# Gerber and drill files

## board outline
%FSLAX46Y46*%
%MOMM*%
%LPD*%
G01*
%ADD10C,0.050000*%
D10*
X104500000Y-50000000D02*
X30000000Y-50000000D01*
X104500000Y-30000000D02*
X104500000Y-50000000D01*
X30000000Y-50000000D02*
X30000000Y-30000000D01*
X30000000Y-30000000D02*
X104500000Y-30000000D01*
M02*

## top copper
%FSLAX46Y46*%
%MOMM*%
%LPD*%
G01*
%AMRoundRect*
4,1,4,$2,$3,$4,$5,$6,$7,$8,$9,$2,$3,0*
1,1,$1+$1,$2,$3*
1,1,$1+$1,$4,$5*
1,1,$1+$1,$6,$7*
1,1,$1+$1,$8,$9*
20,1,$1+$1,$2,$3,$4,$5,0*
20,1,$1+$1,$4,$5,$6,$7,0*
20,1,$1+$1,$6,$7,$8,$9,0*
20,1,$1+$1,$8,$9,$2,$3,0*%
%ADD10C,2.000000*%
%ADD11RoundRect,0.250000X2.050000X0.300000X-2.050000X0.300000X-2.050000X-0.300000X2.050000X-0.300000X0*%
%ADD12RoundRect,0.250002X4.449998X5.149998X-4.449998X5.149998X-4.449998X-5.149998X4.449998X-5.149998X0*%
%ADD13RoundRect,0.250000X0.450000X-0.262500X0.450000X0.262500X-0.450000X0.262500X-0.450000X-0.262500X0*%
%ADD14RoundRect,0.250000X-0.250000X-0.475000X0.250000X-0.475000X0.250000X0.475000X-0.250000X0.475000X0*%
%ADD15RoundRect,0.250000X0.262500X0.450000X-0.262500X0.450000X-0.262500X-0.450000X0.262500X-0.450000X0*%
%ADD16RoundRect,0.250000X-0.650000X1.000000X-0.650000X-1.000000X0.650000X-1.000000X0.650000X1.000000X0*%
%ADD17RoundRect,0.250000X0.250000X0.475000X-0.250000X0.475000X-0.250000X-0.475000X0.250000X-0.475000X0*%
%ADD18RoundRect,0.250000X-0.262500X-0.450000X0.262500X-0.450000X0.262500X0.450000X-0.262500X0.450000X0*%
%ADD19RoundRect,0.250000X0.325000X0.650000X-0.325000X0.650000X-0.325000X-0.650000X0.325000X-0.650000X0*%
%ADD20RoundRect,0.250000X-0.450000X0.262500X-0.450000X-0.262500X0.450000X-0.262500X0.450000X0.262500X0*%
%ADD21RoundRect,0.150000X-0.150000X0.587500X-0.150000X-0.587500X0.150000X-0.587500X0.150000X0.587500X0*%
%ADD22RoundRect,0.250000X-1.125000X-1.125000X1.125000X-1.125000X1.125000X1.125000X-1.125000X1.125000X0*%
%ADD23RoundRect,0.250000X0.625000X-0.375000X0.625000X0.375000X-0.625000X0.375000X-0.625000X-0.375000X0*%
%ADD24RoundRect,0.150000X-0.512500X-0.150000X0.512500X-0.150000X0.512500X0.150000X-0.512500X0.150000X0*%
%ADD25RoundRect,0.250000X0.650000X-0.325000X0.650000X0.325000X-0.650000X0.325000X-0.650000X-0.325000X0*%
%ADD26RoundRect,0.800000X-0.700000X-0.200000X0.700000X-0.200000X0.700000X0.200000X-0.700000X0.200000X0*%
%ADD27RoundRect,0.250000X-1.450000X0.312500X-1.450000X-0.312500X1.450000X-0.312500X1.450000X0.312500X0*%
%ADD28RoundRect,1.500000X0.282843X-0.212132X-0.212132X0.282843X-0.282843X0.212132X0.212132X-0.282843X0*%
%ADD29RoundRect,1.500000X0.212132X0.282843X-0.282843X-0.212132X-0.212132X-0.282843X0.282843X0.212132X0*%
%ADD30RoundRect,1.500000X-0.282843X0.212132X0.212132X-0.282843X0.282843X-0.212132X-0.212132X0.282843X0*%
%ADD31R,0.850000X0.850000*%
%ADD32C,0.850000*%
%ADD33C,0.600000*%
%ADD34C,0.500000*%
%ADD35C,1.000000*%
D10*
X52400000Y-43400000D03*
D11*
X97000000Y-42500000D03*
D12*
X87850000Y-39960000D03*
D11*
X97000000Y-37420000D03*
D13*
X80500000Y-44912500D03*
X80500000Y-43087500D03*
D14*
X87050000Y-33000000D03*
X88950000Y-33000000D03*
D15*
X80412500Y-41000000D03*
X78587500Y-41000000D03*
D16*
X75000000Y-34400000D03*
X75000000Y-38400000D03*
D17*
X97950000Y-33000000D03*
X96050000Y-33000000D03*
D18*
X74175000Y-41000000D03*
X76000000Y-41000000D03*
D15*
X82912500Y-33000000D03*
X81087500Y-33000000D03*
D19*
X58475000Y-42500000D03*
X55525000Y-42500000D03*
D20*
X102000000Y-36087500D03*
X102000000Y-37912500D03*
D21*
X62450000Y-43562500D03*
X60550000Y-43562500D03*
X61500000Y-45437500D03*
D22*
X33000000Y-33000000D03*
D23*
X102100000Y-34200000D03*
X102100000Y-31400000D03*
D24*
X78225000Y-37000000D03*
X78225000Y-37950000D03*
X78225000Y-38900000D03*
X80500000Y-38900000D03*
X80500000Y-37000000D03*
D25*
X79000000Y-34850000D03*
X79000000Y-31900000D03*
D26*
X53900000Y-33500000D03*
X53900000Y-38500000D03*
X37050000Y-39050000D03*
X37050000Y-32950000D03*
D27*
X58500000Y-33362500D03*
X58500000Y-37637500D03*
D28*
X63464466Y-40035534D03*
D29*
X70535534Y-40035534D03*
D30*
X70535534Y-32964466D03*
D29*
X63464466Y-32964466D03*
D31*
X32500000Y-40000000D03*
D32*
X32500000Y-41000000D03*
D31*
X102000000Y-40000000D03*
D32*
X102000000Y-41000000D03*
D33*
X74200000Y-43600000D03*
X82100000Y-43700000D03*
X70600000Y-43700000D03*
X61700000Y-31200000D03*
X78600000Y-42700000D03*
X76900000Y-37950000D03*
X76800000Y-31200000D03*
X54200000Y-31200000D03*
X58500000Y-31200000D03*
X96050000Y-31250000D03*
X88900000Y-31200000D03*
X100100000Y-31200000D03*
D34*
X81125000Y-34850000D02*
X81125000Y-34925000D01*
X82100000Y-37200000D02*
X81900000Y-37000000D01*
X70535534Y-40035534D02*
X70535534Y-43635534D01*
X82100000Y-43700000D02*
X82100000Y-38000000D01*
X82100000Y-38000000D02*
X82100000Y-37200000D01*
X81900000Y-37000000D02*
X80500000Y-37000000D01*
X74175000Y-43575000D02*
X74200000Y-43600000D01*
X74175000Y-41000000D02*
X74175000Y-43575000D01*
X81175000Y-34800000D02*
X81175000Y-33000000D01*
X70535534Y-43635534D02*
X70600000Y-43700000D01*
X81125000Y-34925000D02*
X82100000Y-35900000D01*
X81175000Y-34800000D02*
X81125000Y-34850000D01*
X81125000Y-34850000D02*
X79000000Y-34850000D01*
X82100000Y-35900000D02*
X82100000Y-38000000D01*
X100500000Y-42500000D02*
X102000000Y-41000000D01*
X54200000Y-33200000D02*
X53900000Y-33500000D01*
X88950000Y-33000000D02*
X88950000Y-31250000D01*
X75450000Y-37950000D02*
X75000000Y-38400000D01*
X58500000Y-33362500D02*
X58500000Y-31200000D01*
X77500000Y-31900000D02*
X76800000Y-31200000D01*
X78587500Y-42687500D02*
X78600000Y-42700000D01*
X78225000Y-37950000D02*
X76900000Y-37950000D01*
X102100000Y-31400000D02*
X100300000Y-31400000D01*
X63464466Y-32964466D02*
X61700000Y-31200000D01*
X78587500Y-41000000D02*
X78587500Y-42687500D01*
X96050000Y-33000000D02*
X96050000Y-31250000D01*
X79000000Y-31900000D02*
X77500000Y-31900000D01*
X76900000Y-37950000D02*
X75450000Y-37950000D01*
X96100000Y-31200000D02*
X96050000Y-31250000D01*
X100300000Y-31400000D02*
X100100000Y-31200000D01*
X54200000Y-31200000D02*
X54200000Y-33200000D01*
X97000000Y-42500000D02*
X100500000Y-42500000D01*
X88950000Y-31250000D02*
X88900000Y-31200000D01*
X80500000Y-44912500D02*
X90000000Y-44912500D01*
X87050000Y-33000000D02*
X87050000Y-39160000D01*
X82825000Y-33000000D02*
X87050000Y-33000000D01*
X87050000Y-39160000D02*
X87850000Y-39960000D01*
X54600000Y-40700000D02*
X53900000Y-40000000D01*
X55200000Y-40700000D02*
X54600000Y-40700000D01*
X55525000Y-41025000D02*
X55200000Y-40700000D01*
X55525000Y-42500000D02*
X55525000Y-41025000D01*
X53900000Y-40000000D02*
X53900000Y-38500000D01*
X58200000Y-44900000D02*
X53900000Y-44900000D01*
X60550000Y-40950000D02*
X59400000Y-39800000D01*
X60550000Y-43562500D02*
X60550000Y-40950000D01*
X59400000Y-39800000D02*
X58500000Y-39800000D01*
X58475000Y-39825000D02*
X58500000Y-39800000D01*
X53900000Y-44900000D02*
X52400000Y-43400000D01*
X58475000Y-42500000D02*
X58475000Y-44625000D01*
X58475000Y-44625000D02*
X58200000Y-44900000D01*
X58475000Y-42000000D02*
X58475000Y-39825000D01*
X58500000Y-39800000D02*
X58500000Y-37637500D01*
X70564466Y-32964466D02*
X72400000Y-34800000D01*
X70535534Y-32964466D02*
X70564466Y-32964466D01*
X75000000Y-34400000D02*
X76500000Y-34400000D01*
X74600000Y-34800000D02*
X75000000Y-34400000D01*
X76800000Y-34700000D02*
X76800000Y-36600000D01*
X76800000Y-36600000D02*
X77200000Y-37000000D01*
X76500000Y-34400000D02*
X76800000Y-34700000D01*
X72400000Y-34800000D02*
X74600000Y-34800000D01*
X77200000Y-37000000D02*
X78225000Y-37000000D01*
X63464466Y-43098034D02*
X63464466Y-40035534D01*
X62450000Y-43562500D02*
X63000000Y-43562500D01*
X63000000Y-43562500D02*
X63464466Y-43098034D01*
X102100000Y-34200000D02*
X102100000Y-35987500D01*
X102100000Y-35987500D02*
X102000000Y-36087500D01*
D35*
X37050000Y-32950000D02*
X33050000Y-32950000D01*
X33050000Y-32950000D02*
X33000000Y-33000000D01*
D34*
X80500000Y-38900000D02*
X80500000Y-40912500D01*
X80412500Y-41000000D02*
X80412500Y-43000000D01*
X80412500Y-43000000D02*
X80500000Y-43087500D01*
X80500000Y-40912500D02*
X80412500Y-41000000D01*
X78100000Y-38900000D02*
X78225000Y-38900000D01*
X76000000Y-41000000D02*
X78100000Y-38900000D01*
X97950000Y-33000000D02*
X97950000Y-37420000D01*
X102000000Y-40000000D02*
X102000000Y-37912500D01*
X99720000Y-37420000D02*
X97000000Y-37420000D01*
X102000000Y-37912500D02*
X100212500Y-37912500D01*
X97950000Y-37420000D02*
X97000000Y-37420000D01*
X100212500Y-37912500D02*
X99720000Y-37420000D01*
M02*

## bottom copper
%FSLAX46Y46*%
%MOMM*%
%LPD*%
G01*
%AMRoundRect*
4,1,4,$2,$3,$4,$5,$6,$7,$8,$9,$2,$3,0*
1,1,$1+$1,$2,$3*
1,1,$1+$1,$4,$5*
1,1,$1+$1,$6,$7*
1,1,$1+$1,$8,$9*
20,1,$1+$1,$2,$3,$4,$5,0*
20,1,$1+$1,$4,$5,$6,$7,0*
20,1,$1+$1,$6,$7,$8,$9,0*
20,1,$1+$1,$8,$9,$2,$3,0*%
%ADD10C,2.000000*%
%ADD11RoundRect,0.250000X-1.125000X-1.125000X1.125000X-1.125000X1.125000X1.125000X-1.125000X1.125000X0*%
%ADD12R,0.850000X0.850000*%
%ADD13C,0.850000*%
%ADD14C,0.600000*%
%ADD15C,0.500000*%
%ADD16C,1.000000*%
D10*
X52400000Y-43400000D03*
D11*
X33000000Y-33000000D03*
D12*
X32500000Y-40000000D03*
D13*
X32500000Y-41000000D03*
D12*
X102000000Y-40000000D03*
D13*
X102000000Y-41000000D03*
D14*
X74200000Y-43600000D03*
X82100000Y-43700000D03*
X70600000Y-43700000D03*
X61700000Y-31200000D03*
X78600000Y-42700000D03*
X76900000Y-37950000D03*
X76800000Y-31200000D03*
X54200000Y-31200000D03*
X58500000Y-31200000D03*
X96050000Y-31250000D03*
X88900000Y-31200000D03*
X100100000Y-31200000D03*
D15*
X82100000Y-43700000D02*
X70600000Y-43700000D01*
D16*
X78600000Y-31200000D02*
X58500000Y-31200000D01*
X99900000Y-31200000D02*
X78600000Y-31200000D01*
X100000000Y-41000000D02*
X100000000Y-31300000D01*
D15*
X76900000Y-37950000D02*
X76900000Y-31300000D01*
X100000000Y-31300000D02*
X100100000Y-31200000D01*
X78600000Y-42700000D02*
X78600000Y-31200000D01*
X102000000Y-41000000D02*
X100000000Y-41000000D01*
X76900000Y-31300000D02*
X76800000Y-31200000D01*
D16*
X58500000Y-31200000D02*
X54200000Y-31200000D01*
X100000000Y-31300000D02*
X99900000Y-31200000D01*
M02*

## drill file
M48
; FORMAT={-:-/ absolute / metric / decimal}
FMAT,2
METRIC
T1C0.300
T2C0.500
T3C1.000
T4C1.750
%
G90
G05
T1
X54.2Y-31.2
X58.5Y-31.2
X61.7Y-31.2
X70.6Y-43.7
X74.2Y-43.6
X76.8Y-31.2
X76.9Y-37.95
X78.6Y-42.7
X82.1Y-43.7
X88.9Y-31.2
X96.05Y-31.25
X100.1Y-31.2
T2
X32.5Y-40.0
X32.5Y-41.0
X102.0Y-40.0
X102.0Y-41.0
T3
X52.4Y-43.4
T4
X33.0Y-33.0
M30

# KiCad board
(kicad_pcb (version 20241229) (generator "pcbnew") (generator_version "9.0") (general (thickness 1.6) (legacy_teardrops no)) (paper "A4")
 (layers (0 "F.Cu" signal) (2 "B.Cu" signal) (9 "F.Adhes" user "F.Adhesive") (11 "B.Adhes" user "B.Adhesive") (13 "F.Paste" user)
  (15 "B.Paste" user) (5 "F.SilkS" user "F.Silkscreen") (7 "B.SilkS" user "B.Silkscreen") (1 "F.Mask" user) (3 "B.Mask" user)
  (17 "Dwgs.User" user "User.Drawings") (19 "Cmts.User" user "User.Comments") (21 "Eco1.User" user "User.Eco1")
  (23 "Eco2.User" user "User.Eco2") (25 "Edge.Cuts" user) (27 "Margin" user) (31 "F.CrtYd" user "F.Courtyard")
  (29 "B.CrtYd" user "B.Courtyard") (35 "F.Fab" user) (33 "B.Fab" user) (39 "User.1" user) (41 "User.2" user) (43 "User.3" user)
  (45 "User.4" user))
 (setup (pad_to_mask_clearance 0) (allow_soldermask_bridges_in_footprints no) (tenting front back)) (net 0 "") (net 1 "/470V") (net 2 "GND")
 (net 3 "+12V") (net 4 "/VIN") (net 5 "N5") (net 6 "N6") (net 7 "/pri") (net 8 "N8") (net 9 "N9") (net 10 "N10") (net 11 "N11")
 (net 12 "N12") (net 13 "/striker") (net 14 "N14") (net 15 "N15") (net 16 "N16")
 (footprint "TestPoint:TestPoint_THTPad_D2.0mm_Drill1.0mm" (layer "F.Cu") (at 52.4 43.4)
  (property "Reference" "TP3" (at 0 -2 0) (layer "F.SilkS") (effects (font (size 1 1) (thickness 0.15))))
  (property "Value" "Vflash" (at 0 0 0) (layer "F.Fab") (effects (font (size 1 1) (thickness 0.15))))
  (pad "1" thru_hole circle (at 0 0) (size 2 2) (drill 1) (layers "*.Cu" "*.Mask") (remove_unused_layers no) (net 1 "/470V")))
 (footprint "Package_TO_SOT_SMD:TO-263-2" (layer "F.Cu") (at 89.35 39.96 180)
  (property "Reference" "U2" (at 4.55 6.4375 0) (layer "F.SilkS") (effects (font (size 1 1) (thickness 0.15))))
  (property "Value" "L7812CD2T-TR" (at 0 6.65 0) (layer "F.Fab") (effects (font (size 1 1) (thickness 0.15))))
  (pad "" smd roundrect (at -0.925 -2.775 180) (size 4.55 5.25) (layers "F.Paste") (roundrect_rratio 0.054945))
  (pad "" smd roundrect (at -0.925 2.775 180) (size 4.55 5.25) (layers "F.Paste") (roundrect_rratio 0.054945))
  (pad "" smd roundrect (at 3.925 -2.775 180) (size 4.55 5.25) (layers "F.Paste") (roundrect_rratio 0.054945))
  (pad "" smd roundrect (at 3.925 2.775 180) (size 4.55 5.25) (layers "F.Paste") (roundrect_rratio 0.054945))
  (pad "1" smd roundrect (at -7.65 -2.54 180) (size 4.6 1.1) (layers "F.Cu" "F.Mask" "F.Paste") (roundrect_rratio 0.227273) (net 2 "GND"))
  (pad "2" smd roundrect (at 1.5 0 180) (size 9.4 10.8) (layers "F.Cu" "F.Mask") (roundrect_rratio 0.026596) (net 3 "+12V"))
  (pad "3" smd roundrect (at -7.65 2.54 180) (size 4.6 1.1) (layers "F.Cu" "F.Mask" "F.Paste") (roundrect_rratio 0.227273) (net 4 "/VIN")))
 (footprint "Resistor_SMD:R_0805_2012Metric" (layer "F.Cu") (at 80.5 44 90)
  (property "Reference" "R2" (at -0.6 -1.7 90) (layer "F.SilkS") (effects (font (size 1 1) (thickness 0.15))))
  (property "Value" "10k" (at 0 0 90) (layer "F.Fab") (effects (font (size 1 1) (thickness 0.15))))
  (pad "1" smd roundrect (at -0.9125 0 90) (size 1.025 1.4) (layers "F.Cu" "F.Mask" "F.Paste") (roundrect_rratio 0.243902) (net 3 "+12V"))
  (pad "2" smd roundrect (at 0.9125 0 90) (size 1.025 1.4) (layers "F.Cu" "F.Mask" "F.Paste") (roundrect_rratio 0.243902) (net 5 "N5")))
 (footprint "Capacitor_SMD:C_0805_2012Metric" (layer "F.Cu") (at 88 33)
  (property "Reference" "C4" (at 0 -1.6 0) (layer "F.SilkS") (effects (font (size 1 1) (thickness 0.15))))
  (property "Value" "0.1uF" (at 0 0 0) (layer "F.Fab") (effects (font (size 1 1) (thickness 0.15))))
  (pad "1" smd roundrect (at -0.95 0) (size 1 1.45) (layers "F.Cu" "F.Mask" "F.Paste") (roundrect_rratio 0.25) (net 3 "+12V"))
  (pad "2" smd roundrect (at 0.95 0) (size 1 1.45) (layers "F.Cu" "F.Mask" "F.Paste") (roundrect_rratio 0.25) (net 2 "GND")))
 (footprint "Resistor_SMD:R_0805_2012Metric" (layer "F.Cu") (at 79.5 41 180)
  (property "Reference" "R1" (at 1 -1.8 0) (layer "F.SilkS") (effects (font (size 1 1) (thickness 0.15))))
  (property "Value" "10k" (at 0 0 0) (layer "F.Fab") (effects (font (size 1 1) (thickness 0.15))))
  (pad "1" smd roundrect (at -0.9125 0 180) (size 1.025 1.4) (layers "F.Cu" "F.Mask" "F.Paste") (roundrect_rratio 0.243902) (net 5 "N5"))
  (pad "2" smd roundrect (at 0.9125 0 180) (size 1.025 1.4) (layers "F.Cu" "F.Mask" "F.Paste") (roundrect_rratio 0.243902) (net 2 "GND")))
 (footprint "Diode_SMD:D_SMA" (layer "F.Cu") (at 75 36.4 -90)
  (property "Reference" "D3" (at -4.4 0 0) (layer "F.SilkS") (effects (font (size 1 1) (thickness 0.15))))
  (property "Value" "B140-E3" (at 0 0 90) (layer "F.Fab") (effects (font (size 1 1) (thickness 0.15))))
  (pad "1" smd roundrect (at -2 0 270) (size 2.5 1.8) (layers "F.Cu" "F.Mask" "F.Paste") (roundrect_rratio 0.1388888889) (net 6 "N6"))
  (pad "2" smd roundrect (at 2 0 270) (size 2.5 1.8) (layers "F.Cu" "F.Mask" "F.Paste") (roundrect_rratio 0.1388888889) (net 2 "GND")))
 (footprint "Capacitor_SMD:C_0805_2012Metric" (layer "F.Cu") (at 97 33 180)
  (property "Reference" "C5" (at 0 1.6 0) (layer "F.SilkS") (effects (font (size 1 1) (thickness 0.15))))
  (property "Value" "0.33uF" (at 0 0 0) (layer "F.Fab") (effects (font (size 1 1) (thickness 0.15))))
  (pad "1" smd roundrect (at -0.95 0 180) (size 1 1.45) (layers "F.Cu" "F.Mask" "F.Paste") (roundrect_rratio 0.25) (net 4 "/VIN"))
  (pad "2" smd roundrect (at 0.95 0 180) (size 1 1.45) (layers "F.Cu" "F.Mask" "F.Paste") (roundrect_rratio 0.25) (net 2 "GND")))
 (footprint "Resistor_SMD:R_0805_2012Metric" (layer "F.Cu") (at 75.0875 41)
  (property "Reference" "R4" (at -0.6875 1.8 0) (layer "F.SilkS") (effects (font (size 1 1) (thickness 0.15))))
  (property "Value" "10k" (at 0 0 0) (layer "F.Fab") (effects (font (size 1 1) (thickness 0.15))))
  (pad "1" smd roundrect (at -0.9125 0) (size 1.025 1.4) (layers "F.Cu" "F.Mask" "F.Paste") (roundrect_rratio 0.243902) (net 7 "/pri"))
  (pad "2" smd roundrect (at 0.9125 0) (size 1.025 1.4) (layers "F.Cu" "F.Mask" "F.Paste") (roundrect_rratio 0.243902) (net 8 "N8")))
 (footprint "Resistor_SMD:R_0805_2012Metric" (layer "F.Cu") (at 82 33 180)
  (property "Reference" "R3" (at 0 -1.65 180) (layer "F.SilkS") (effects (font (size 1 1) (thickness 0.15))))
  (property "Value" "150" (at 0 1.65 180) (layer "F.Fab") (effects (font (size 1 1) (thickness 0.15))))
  (pad "1" smd roundrect (at -0.9125 0 180) (size 1.025 1.4) (layers "F.Cu" "F.Mask" "F.Paste") (roundrect_rratio 0.243902) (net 3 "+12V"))
  (pad "2" smd roundrect (at 0.9125 0 180) (size 1.025 1.4) (layers "F.Cu" "F.Mask" "F.Paste") (roundrect_rratio 0.243902) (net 7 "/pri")))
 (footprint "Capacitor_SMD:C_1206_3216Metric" (layer "F.Cu") (at 57 42.5 180)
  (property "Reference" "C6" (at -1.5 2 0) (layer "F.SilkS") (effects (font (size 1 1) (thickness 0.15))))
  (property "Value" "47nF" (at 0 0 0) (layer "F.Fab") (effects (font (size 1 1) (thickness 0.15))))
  (pad "1" smd roundrect (at -1.475 0 180) (size 1.15 1.8) (layers "F.Cu" "F.Mask" "F.Paste") (roundrect_rratio 0.217391) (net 1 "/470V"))
  (pad "2" smd roundrect (at 1.475 0 180) (size 1.15 1.8) (layers "F.Cu" "F.Mask" "F.Paste") (roundrect_rratio 0.217391) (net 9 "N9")))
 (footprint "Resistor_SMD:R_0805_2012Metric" (layer "F.Cu") (at 102 37 -90)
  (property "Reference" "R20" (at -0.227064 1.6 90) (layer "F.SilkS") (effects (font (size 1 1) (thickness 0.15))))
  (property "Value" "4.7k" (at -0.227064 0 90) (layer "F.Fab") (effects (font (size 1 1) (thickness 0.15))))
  (pad "1" smd roundrect (at -0.9125 0 270) (size 1.025 1.4) (layers "F.Cu" "F.Mask" "F.Paste") (roundrect_rratio 0.243902) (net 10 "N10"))
  (pad "2" smd roundrect (at 0.9125 0 270) (size 1.025 1.4) (layers "F.Cu" "F.Mask" "F.Paste") (roundrect_rratio 0.243902) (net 4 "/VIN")))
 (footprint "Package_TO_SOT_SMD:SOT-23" (layer "F.Cu") (at 61.5 44.5 -90)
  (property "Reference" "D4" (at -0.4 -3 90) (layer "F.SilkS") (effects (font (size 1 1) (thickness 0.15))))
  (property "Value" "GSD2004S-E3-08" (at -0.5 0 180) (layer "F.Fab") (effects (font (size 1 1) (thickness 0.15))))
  (pad "1" smd roundrect (at -0.9375 -0.95 270) (size 1.475 0.6) (layers "F.Cu" "F.Mask" "F.Paste") (roundrect_rratio 0.25) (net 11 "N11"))
  (pad "2" smd roundrect (at -0.9375 0.95 270) (size 1.475 0.6) (layers "F.Cu" "F.Mask" "F.Paste") (roundrect_rratio 0.25) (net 1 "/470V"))
  (pad "3" smd roundrect (at 0.9375 0 270) (size 1.475 0.6) (layers "F.Cu" "F.Mask" "F.Paste") (roundrect_rratio 0.25) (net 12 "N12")))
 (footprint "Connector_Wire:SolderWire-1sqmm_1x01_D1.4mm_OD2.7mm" (layer "F.Cu") (at 33 33)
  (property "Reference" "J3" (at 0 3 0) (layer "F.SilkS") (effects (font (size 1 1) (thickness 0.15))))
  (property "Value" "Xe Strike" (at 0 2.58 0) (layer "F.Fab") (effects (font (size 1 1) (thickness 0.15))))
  (pad "1" thru_hole roundrect (at 0 0) (size 2.75 2.75) (drill 1.75) (layers "*.Cu" "*.Mask") (remove_unused_layers no)
   (roundrect_rratio 0.090909) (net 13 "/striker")))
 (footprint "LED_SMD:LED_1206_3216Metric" (layer "F.Cu") (at 102.1 32.8 90)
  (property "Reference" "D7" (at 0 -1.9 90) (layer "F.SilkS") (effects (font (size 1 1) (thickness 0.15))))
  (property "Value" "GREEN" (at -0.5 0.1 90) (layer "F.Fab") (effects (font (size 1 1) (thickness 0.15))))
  (pad "1" smd roundrect (at -1.4 0 90) (size 1.25 1.75) (layers "F.Cu" "F.Mask" "F.Paste") (roundrect_rratio 0.2) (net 10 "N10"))
  (pad "2" smd roundrect (at 1.4 0 90) (size 1.25 1.75) (layers "F.Cu" "F.Mask" "F.Paste") (roundrect_rratio 0.2) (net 2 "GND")))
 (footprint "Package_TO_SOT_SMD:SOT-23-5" (layer "F.Cu") (at 79.3625 37.95)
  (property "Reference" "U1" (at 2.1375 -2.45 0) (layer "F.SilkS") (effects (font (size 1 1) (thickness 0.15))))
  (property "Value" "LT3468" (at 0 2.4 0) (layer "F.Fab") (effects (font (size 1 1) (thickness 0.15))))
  (pad "1" smd roundrect (at -1.1375 -0.95) (size 1.325 0.6) (layers "F.Cu" "F.Mask" "F.Paste") (roundrect_rratio 0.25) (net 6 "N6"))
  (pad "2" smd roundrect (at -1.1375 0) (size 1.325 0.6) (layers "F.Cu" "F.Mask" "F.Paste") (roundrect_rratio 0.25) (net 2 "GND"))
  (pad "3" smd roundrect (at -1.1375 0.95) (size 1.325 0.6) (layers "F.Cu" "F.Mask" "F.Paste") (roundrect_rratio 0.25) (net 8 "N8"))
  (pad "4" smd roundrect (at 1.1375 0.95) (size 1.325 0.6) (layers "F.Cu" "F.Mask" "F.Paste") (roundrect_rratio 0.25) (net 5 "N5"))
  (pad "5" smd roundrect (at 1.1375 -0.95) (size 1.325 0.6) (layers "F.Cu" "F.Mask" "F.Paste") (roundrect_rratio 0.25) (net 7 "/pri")))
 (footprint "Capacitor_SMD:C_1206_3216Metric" (layer "F.Cu") (at 79 33.375 90)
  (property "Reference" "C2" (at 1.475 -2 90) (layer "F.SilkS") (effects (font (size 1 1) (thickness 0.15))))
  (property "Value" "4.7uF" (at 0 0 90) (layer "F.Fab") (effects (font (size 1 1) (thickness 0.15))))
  (pad "1" smd roundrect (at -1.475 0 90) (size 1.15 1.8) (layers "F.Cu" "F.Mask" "F.Paste") (roundrect_rratio 0.217391) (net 7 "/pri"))
  (pad "2" smd roundrect (at 1.475 0 90) (size 1.15 1.8) (layers "F.Cu" "F.Mask" "F.Paste") (roundrect_rratio 0.217391) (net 2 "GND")))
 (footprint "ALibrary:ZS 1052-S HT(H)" (layer "F.Cu") (at 45.5 36 180)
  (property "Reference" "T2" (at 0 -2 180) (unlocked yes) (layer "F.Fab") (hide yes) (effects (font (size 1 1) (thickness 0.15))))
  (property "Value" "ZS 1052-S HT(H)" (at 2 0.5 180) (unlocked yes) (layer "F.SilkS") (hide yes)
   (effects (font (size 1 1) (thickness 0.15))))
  (pad "1" smd roundrect (at -8.4 2.5) (size 3 2) (layers "F.Cu" "F.Mask" "F.Paste") (roundrect_rratio 0.4) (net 2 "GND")
   (thermal_bridge_angle 45))
  (pad "2" smd roundrect (at -8.4 -2.5) (size 3 2) (layers "F.Cu" "F.Mask" "F.Paste") (roundrect_rratio 0.4) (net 9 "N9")
   (thermal_bridge_angle 45))
  (pad "3" smd roundrect (at 8.45 -3.05) (size 3 2) (layers "F.Cu" "F.Mask" "F.Paste") (roundrect_rratio 0.4) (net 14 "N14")
   (thermal_bridge_angle 45))
  (pad "4" smd roundrect (at 8.45 3.05) (size 3 2) (layers "F.Cu" "F.Mask" "F.Paste") (roundrect_rratio 0.4) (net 13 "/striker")
   (thermal_bridge_angle 45)))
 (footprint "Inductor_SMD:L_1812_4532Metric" (layer "F.Cu") (at 58.5 35.5 -90)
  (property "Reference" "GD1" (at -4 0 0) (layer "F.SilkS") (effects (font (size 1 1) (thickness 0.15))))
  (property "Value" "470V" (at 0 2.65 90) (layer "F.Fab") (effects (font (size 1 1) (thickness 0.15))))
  (pad "1" smd roundrect (at -2.1375 0 270) (size 1.125 3.4) (layers "F.Cu" "F.Mask" "F.Paste") (roundrect_rratio 0.222222) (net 2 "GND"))
  (pad "2" smd roundrect (at 2.1375 0 270) (size 1.125 3.4) (layers "F.Cu" "F.Mask" "F.Paste") (roundrect_rratio 0.222222) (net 1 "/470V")))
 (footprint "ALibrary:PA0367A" (layer "F.Cu") (at 67 36.5 135)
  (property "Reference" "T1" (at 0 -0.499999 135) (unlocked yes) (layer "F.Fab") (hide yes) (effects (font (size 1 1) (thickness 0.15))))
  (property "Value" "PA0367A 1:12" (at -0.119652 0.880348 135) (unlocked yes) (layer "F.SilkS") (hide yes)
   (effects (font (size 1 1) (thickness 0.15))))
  (pad "1" smd roundrect (at 0 -5 135) (size 3.7 3.1) (layers "F.Cu" "F.Mask" "F.Paste") (roundrect_rratio 0.4838709677) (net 11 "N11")
   (thermal_bridge_angle 45))
  (pad "2" smd roundrect (at -5 0 225) (size 3.7 3.1) (layers "F.Cu" "F.Mask" "F.Paste") (roundrect_rratio 0.4838709677) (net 7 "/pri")
   (thermal_bridge_angle 45))
  (pad "3" smd roundrect (at 0 5 315) (size 3.7 3.1) (layers "F.Cu" "F.Mask" "F.Paste") (roundrect_rratio 0.4838709677) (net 6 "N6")
   (thermal_bridge_angle 45))
  (pad "4" smd roundrect (at 5 0 225) (size 3.7 3.1) (layers "F.Cu" "F.Mask" "F.Paste") (roundrect_rratio 0.4838709677) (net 2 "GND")
   (thermal_bridge_angle 45)))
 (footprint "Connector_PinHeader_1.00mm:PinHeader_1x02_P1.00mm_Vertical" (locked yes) (layer "B.Cu") (at 32.5 40 180)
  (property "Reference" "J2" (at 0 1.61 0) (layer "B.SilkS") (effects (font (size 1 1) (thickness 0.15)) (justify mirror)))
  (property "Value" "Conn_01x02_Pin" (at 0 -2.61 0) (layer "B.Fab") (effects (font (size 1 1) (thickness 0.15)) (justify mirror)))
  (pad "1" thru_hole rect (at 0 0 180) (size 0.85 0.85) (drill 0.5) (layers "*.Cu" "*.Mask") (remove_unused_layers no) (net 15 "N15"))
  (pad "2" thru_hole circle (at 0 -1 180) (size 0.85 0.85) (drill 0.5) (layers "*.Cu" "*.Mask") (remove_unused_layers no) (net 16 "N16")))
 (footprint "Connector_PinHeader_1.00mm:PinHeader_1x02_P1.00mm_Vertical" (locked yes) (layer "B.Cu") (at 102 40 180)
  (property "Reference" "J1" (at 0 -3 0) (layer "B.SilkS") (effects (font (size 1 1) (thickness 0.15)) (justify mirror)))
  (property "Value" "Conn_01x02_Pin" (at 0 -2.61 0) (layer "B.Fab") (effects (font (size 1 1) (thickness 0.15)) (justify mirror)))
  (pad "1" thru_hole rect (at 0 0 180) (size 0.85 0.85) (drill 0.5) (layers "*.Cu" "*.Mask") (remove_unused_layers no) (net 4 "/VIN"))
  (pad "2" thru_hole circle (at 0 -1 180) (size 0.85 0.85) (drill 0.5) (layers "*.Cu" "*.Mask") (remove_unused_layers no) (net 2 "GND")))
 (gr_line (start 104.5 50) (end 30 50) (stroke (width 0.05) (type default)) (layer "Edge.Cuts"))
 (gr_line (start 104.5 30) (end 104.5 50) (stroke (width 0.05) (type default)) (layer "Edge.Cuts"))
 (gr_line (start 30 50) (end 30 30) (stroke (width 0.05) (type default)) (layer "Edge.Cuts"))
 (gr_line (start 30 30) (end 104.5 30) (stroke (width 0.05) (type default)) (layer "Edge.Cuts"))
 (segment (start 81.125 34.85) (end 81.125 34.925) (width 0.5) (layer "F.Cu") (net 7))
 (segment (start 82.1 37.2) (end 81.9 37) (width 0.5) (layer "F.Cu") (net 7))
 (segment (start 70.535534 40.035534) (end 70.535534 43.635534) (width 0.5) (layer "F.Cu") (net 7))
 (segment (start 82.1 43.7) (end 82.1 38) (width 0.5) (layer "F.Cu") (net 7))
 (segment (start 82.1 38) (end 82.1 37.2) (width 0.5) (layer "F.Cu") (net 7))
 (segment (start 81.9 37) (end 80.5 37) (width 0.5) (layer "F.Cu") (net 7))
 (segment (start 74.175 43.575) (end 74.2 43.6) (width 0.5) (layer "F.Cu") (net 7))
 (segment (start 74.175 41) (end 74.175 43.575) (width 0.5) (layer "F.Cu") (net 7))
 (segment (start 81.175 34.8) (end 81.175 33) (width 0.5) (layer "F.Cu") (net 7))
 (segment (start 70.535534 43.635534) (end 70.6 43.7) (width 0.5) (layer "F.Cu") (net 7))
 (segment (start 81.125 34.925) (end 82.1 35.9) (width 0.5) (layer "F.Cu") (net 7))
 (segment (start 81.175 34.8) (end 81.125 34.85) (width 0.5) (layer "F.Cu") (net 7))
 (segment (start 81.125 34.85) (end 79 34.85) (width 0.5) (layer "F.Cu") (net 7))
 (segment (start 82.1 35.9) (end 82.1 38) (width 0.5) (layer "F.Cu") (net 7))
 (via (at 74.2 43.6) (size 0.6) (drill 0.3) (layers "F.Cu" "B.Cu") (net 7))
 (via (at 82.1 43.7) (size 0.6) (drill 0.3) (layers "F.Cu" "B.Cu") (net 7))
 (via (at 70.6 43.7) (size 0.6) (drill 0.3) (layers "F.Cu" "B.Cu") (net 7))
 (segment (start 82.1 43.7) (end 70.6 43.7) (width 0.5) (layer "B.Cu") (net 7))
 (segment (start 100.5 42.5) (end 102 41) (width 0.5) (layer "F.Cu") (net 2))
 (segment (start 54.2 33.2) (end 53.9 33.5) (width 0.5) (layer "F.Cu") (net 2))
 (segment (start 88.95 33) (end 88.95 31.25) (width 0.5) (layer "F.Cu") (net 2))
 (segment (start 75.45 37.95) (end 75 38.4) (width 0.5) (layer "F.Cu") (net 2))
 (segment (start 58.5 33.3625) (end 58.5 31.2) (width 0.5) (layer "F.Cu") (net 2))
 (segment (start 77.5 31.9) (end 76.8 31.2) (width 0.5) (layer "F.Cu") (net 2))
 (segment (start 78.5875 42.6875) (end 78.6 42.7) (width 0.5) (layer "F.Cu") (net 2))
 (segment (start 78.225 37.95) (end 76.9 37.95) (width 0.5) (layer "F.Cu") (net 2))
 (segment (start 102.1 31.4) (end 100.3 31.4) (width 0.5) (layer "F.Cu") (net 2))
 (segment (start 63.464466 32.964466) (end 61.7 31.2) (width 0.5) (layer "F.Cu") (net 2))
 (segment (start 78.5875 41) (end 78.5875 42.6875) (width 0.5) (layer "F.Cu") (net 2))
 (segment (start 96.05 33) (end 96.05 31.25) (width 0.5) (layer "F.Cu") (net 2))
 (segment (start 79 31.9) (end 77.5 31.9) (width 0.5) (layer "F.Cu") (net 2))
 (segment (start 76.9 37.95) (end 75.45 37.95) (width 0.5) (layer "F.Cu") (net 2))
 (segment (start 96.1 31.2) (end 96.05 31.25) (width 0.5) (layer "F.Cu") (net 2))
 (segment (start 100.3 31.4) (end 100.1 31.2) (width 0.5) (layer "F.Cu") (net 2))
 (segment (start 54.2 31.2) (end 54.2 33.2) (width 0.5) (layer "F.Cu") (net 2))
 (segment (start 97 42.5) (end 100.5 42.5) (width 0.5) (layer "F.Cu") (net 2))
 (segment (start 88.95 31.25) (end 88.9 31.2) (width 0.5) (layer "F.Cu") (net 2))
 (via (at 61.7 31.2) (size 0.6) (drill 0.3) (layers "F.Cu" "B.Cu") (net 2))
 (via (at 78.6 42.7) (size 0.6) (drill 0.3) (layers "F.Cu" "B.Cu") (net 2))
 (via (at 76.9 37.95) (size 0.6) (drill 0.3) (layers "F.Cu" "B.Cu") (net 2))
 (via (at 76.8 31.2) (size 0.6) (drill 0.3) (layers "F.Cu" "B.Cu") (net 2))
 (via (at 54.2 31.2) (size 0.6) (drill 0.3) (layers "F.Cu" "B.Cu") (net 2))
 (via (at 58.5 31.2) (size 0.6) (drill 0.3) (layers "F.Cu" "B.Cu") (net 2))
 (via (at 96.05 31.25) (size 0.6) (drill 0.3) (layers "F.Cu" "B.Cu") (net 2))
 (via (at 88.9 31.2) (size 0.6) (drill 0.3) (layers "F.Cu" "B.Cu") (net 2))
 (via (at 100.1 31.2) (size 0.6) (drill 0.3) (layers "F.Cu" "B.Cu") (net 2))
 (segment (start 78.6 31.2) (end 58.5 31.2) (width 1) (layer "B.Cu") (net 2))
 (segment (start 99.9 31.2) (end 78.6 31.2) (width 1) (layer "B.Cu") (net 2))
 (segment (start 100 41) (end 100 31.3) (width 1) (layer "B.Cu") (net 2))
 (segment (start 76.9 37.95) (end 76.9 31.3) (width 0.5) (layer "B.Cu") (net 2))
 (segment (start 100 31.3) (end 100.1 31.2) (width 0.5) (layer "B.Cu") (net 2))
 (segment (start 78.6 42.7) (end 78.6 31.2) (width 0.5) (layer "B.Cu") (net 2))
 (segment (start 102 41) (end 100 41) (width 0.5) (layer "B.Cu") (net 2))
 (segment (start 76.9 31.3) (end 76.8 31.2) (width 0.5) (layer "B.Cu") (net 2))
 (segment (start 58.5 31.2) (end 54.2 31.2) (width 1) (layer "B.Cu") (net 2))
 (segment (start 100 31.3) (end 99.9 31.2) (width 1) (layer "B.Cu") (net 2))
 (segment (start 80.5 44.9125) (end 90 44.9125) (width 0.5) (layer "F.Cu") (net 3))
 (segment (start 87.05 33) (end 87.05 39.16) (width 0.5) (layer "F.Cu") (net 3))
 (segment (start 82.825 33) (end 87.05 33) (width 0.5) (layer "F.Cu") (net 3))
 (segment (start 87.05 39.16) (end 87.85 39.96) (width 0.5) (layer "F.Cu") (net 3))
 (segment (start 54.6 40.7) (end 53.9 40) (width 0.5) (layer "F.Cu") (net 9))
 (segment (start 55.2 40.7) (end 54.6 40.7) (width 0.5) (layer "F.Cu") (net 9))
 (segment (start 55.525 41.025) (end 55.2 40.7) (width 0.5) (layer "F.Cu") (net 9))
 (segment (start 55.525 42.5) (end 55.525 41.025) (width 0.5) (layer "F.Cu") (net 9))
 (segment (start 53.9 40) (end 53.9 38.5) (width 0.5) (layer "F.Cu") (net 9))
 (segment (start 58.2 44.9) (end 53.9 44.9) (width 0.5) (layer "F.Cu") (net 1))
 (segment (start 60.55 40.95) (end 59.4 39.8) (width 0.5) (layer "F.Cu") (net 1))
 (segment (start 60.55 43.5625) (end 60.55 40.95) (width 0.5) (layer "F.Cu") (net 1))
 (segment (start 59.4 39.8) (end 58.5 39.8) (width 0.5) (layer "F.Cu") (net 1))
 (segment (start 58.475 39.825) (end 58.5 39.8) (width 0.5) (layer "F.Cu") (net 1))
 (segment (start 53.9 44.9) (end 52.4 43.4) (width 0.5) (layer "F.Cu") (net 1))
 (segment (start 58.475 42.5) (end 58.475 44.625) (width 0.5) (layer "F.Cu") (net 1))
 (segment (start 58.475 44.625) (end 58.2 44.9) (width 0.5) (layer "F.Cu") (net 1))
 (segment (start 58.475 42) (end 58.475 39.825) (width 0.5) (layer "F.Cu") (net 1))
 (segment (start 58.5 39.8) (end 58.5 37.6375) (width 0.5) (layer "F.Cu") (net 1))
 (segment (start 70.564466 32.964466) (end 72.4 34.8) (width 0.5) (layer "F.Cu") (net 6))
 (segment (start 70.535534 32.964466) (end 70.564466 32.964466) (width 0.5) (layer "F.Cu") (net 6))
 (segment (start 75 34.4) (end 76.5 34.4) (width 0.5) (layer "F.Cu") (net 6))
 (segment (start 74.6 34.8) (end 75 34.4) (width 0.5) (layer "F.Cu") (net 6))
 (segment (start 76.8 34.7) (end 76.8 36.6) (width 0.5) (layer "F.Cu") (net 6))
 (segment (start 76.8 36.6) (end 77.2 37) (width 0.5) (layer "F.Cu") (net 6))
 (segment (start 76.5 34.4) (end 76.8 34.7) (width 0.5) (layer "F.Cu") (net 6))
 (segment (start 72.4 34.8) (end 74.6 34.8) (width 0.5) (layer "F.Cu") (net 6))
 (segment (start 77.2 37) (end 78.225 37) (width 0.5) (layer "F.Cu") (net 6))
 (segment (start 63.464466 43.098034) (end 63.464466 40.035534) (width 0.5) (layer "F.Cu") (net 11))
 (segment (start 62.45 43.5625) (end 63 43.5625) (width 0.5) (layer "F.Cu") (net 11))
 (segment (start 63 43.5625) (end 63.464466 43.098034) (width 0.5) (layer "F.Cu") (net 11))
 (segment (start 102.1 34.2) (end 102.1 35.9875) (width 0.5) (layer "F.Cu") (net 10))
 (segment (start 102.1 35.9875) (end 102 36.0875) (width 0.5) (layer "F.Cu") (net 10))
 (segment (start 37.05 32.95) (end 33.05 32.95) (width 1) (layer "F.Cu") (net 13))
 (segment (start 33.05 32.95) (end 33 33) (width 1) (layer "F.Cu") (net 13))
 (segment (start 80.5 38.9) (end 80.5 40.9125) (width 0.5) (layer "F.Cu") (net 5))
 (segment (start 80.4125 41) (end 80.4125 43) (width 0.5) (layer "F.Cu") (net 5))
 (segment (start 80.4125 43) (end 80.5 43.0875) (width 0.5) (layer "F.Cu") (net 5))
 (segment (start 80.5 40.9125) (end 80.4125 41) (width 0.5) (layer "F.Cu") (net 5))
 (segment (start 78.1 38.9) (end 78.225 38.9) (width 0.5) (layer "F.Cu") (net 8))
 (segment (start 76 41) (end 78.1 38.9) (width 0.5) (layer "F.Cu") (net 8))
 (segment (start 97.95 33) (end 97.95 37.42) (width 0.5) (layer "F.Cu") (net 4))
 (segment (start 102 40) (end 102 37.9125) (width 0.5) (layer "F.Cu") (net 4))
 (segment (start 99.72 37.42) (end 97 37.42) (width 0.5) (layer "F.Cu") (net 4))
 (segment (start 102 37.9125) (end 100.2125 37.9125) (width 0.5) (layer "F.Cu") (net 4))
 (segment (start 97.95 37.42) (end 97 37.42) (width 0.5) (layer "F.Cu") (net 4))
 (segment (start 100.2125 37.9125) (end 99.72 37.42) (width 0.5) (layer "F.Cu") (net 4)))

